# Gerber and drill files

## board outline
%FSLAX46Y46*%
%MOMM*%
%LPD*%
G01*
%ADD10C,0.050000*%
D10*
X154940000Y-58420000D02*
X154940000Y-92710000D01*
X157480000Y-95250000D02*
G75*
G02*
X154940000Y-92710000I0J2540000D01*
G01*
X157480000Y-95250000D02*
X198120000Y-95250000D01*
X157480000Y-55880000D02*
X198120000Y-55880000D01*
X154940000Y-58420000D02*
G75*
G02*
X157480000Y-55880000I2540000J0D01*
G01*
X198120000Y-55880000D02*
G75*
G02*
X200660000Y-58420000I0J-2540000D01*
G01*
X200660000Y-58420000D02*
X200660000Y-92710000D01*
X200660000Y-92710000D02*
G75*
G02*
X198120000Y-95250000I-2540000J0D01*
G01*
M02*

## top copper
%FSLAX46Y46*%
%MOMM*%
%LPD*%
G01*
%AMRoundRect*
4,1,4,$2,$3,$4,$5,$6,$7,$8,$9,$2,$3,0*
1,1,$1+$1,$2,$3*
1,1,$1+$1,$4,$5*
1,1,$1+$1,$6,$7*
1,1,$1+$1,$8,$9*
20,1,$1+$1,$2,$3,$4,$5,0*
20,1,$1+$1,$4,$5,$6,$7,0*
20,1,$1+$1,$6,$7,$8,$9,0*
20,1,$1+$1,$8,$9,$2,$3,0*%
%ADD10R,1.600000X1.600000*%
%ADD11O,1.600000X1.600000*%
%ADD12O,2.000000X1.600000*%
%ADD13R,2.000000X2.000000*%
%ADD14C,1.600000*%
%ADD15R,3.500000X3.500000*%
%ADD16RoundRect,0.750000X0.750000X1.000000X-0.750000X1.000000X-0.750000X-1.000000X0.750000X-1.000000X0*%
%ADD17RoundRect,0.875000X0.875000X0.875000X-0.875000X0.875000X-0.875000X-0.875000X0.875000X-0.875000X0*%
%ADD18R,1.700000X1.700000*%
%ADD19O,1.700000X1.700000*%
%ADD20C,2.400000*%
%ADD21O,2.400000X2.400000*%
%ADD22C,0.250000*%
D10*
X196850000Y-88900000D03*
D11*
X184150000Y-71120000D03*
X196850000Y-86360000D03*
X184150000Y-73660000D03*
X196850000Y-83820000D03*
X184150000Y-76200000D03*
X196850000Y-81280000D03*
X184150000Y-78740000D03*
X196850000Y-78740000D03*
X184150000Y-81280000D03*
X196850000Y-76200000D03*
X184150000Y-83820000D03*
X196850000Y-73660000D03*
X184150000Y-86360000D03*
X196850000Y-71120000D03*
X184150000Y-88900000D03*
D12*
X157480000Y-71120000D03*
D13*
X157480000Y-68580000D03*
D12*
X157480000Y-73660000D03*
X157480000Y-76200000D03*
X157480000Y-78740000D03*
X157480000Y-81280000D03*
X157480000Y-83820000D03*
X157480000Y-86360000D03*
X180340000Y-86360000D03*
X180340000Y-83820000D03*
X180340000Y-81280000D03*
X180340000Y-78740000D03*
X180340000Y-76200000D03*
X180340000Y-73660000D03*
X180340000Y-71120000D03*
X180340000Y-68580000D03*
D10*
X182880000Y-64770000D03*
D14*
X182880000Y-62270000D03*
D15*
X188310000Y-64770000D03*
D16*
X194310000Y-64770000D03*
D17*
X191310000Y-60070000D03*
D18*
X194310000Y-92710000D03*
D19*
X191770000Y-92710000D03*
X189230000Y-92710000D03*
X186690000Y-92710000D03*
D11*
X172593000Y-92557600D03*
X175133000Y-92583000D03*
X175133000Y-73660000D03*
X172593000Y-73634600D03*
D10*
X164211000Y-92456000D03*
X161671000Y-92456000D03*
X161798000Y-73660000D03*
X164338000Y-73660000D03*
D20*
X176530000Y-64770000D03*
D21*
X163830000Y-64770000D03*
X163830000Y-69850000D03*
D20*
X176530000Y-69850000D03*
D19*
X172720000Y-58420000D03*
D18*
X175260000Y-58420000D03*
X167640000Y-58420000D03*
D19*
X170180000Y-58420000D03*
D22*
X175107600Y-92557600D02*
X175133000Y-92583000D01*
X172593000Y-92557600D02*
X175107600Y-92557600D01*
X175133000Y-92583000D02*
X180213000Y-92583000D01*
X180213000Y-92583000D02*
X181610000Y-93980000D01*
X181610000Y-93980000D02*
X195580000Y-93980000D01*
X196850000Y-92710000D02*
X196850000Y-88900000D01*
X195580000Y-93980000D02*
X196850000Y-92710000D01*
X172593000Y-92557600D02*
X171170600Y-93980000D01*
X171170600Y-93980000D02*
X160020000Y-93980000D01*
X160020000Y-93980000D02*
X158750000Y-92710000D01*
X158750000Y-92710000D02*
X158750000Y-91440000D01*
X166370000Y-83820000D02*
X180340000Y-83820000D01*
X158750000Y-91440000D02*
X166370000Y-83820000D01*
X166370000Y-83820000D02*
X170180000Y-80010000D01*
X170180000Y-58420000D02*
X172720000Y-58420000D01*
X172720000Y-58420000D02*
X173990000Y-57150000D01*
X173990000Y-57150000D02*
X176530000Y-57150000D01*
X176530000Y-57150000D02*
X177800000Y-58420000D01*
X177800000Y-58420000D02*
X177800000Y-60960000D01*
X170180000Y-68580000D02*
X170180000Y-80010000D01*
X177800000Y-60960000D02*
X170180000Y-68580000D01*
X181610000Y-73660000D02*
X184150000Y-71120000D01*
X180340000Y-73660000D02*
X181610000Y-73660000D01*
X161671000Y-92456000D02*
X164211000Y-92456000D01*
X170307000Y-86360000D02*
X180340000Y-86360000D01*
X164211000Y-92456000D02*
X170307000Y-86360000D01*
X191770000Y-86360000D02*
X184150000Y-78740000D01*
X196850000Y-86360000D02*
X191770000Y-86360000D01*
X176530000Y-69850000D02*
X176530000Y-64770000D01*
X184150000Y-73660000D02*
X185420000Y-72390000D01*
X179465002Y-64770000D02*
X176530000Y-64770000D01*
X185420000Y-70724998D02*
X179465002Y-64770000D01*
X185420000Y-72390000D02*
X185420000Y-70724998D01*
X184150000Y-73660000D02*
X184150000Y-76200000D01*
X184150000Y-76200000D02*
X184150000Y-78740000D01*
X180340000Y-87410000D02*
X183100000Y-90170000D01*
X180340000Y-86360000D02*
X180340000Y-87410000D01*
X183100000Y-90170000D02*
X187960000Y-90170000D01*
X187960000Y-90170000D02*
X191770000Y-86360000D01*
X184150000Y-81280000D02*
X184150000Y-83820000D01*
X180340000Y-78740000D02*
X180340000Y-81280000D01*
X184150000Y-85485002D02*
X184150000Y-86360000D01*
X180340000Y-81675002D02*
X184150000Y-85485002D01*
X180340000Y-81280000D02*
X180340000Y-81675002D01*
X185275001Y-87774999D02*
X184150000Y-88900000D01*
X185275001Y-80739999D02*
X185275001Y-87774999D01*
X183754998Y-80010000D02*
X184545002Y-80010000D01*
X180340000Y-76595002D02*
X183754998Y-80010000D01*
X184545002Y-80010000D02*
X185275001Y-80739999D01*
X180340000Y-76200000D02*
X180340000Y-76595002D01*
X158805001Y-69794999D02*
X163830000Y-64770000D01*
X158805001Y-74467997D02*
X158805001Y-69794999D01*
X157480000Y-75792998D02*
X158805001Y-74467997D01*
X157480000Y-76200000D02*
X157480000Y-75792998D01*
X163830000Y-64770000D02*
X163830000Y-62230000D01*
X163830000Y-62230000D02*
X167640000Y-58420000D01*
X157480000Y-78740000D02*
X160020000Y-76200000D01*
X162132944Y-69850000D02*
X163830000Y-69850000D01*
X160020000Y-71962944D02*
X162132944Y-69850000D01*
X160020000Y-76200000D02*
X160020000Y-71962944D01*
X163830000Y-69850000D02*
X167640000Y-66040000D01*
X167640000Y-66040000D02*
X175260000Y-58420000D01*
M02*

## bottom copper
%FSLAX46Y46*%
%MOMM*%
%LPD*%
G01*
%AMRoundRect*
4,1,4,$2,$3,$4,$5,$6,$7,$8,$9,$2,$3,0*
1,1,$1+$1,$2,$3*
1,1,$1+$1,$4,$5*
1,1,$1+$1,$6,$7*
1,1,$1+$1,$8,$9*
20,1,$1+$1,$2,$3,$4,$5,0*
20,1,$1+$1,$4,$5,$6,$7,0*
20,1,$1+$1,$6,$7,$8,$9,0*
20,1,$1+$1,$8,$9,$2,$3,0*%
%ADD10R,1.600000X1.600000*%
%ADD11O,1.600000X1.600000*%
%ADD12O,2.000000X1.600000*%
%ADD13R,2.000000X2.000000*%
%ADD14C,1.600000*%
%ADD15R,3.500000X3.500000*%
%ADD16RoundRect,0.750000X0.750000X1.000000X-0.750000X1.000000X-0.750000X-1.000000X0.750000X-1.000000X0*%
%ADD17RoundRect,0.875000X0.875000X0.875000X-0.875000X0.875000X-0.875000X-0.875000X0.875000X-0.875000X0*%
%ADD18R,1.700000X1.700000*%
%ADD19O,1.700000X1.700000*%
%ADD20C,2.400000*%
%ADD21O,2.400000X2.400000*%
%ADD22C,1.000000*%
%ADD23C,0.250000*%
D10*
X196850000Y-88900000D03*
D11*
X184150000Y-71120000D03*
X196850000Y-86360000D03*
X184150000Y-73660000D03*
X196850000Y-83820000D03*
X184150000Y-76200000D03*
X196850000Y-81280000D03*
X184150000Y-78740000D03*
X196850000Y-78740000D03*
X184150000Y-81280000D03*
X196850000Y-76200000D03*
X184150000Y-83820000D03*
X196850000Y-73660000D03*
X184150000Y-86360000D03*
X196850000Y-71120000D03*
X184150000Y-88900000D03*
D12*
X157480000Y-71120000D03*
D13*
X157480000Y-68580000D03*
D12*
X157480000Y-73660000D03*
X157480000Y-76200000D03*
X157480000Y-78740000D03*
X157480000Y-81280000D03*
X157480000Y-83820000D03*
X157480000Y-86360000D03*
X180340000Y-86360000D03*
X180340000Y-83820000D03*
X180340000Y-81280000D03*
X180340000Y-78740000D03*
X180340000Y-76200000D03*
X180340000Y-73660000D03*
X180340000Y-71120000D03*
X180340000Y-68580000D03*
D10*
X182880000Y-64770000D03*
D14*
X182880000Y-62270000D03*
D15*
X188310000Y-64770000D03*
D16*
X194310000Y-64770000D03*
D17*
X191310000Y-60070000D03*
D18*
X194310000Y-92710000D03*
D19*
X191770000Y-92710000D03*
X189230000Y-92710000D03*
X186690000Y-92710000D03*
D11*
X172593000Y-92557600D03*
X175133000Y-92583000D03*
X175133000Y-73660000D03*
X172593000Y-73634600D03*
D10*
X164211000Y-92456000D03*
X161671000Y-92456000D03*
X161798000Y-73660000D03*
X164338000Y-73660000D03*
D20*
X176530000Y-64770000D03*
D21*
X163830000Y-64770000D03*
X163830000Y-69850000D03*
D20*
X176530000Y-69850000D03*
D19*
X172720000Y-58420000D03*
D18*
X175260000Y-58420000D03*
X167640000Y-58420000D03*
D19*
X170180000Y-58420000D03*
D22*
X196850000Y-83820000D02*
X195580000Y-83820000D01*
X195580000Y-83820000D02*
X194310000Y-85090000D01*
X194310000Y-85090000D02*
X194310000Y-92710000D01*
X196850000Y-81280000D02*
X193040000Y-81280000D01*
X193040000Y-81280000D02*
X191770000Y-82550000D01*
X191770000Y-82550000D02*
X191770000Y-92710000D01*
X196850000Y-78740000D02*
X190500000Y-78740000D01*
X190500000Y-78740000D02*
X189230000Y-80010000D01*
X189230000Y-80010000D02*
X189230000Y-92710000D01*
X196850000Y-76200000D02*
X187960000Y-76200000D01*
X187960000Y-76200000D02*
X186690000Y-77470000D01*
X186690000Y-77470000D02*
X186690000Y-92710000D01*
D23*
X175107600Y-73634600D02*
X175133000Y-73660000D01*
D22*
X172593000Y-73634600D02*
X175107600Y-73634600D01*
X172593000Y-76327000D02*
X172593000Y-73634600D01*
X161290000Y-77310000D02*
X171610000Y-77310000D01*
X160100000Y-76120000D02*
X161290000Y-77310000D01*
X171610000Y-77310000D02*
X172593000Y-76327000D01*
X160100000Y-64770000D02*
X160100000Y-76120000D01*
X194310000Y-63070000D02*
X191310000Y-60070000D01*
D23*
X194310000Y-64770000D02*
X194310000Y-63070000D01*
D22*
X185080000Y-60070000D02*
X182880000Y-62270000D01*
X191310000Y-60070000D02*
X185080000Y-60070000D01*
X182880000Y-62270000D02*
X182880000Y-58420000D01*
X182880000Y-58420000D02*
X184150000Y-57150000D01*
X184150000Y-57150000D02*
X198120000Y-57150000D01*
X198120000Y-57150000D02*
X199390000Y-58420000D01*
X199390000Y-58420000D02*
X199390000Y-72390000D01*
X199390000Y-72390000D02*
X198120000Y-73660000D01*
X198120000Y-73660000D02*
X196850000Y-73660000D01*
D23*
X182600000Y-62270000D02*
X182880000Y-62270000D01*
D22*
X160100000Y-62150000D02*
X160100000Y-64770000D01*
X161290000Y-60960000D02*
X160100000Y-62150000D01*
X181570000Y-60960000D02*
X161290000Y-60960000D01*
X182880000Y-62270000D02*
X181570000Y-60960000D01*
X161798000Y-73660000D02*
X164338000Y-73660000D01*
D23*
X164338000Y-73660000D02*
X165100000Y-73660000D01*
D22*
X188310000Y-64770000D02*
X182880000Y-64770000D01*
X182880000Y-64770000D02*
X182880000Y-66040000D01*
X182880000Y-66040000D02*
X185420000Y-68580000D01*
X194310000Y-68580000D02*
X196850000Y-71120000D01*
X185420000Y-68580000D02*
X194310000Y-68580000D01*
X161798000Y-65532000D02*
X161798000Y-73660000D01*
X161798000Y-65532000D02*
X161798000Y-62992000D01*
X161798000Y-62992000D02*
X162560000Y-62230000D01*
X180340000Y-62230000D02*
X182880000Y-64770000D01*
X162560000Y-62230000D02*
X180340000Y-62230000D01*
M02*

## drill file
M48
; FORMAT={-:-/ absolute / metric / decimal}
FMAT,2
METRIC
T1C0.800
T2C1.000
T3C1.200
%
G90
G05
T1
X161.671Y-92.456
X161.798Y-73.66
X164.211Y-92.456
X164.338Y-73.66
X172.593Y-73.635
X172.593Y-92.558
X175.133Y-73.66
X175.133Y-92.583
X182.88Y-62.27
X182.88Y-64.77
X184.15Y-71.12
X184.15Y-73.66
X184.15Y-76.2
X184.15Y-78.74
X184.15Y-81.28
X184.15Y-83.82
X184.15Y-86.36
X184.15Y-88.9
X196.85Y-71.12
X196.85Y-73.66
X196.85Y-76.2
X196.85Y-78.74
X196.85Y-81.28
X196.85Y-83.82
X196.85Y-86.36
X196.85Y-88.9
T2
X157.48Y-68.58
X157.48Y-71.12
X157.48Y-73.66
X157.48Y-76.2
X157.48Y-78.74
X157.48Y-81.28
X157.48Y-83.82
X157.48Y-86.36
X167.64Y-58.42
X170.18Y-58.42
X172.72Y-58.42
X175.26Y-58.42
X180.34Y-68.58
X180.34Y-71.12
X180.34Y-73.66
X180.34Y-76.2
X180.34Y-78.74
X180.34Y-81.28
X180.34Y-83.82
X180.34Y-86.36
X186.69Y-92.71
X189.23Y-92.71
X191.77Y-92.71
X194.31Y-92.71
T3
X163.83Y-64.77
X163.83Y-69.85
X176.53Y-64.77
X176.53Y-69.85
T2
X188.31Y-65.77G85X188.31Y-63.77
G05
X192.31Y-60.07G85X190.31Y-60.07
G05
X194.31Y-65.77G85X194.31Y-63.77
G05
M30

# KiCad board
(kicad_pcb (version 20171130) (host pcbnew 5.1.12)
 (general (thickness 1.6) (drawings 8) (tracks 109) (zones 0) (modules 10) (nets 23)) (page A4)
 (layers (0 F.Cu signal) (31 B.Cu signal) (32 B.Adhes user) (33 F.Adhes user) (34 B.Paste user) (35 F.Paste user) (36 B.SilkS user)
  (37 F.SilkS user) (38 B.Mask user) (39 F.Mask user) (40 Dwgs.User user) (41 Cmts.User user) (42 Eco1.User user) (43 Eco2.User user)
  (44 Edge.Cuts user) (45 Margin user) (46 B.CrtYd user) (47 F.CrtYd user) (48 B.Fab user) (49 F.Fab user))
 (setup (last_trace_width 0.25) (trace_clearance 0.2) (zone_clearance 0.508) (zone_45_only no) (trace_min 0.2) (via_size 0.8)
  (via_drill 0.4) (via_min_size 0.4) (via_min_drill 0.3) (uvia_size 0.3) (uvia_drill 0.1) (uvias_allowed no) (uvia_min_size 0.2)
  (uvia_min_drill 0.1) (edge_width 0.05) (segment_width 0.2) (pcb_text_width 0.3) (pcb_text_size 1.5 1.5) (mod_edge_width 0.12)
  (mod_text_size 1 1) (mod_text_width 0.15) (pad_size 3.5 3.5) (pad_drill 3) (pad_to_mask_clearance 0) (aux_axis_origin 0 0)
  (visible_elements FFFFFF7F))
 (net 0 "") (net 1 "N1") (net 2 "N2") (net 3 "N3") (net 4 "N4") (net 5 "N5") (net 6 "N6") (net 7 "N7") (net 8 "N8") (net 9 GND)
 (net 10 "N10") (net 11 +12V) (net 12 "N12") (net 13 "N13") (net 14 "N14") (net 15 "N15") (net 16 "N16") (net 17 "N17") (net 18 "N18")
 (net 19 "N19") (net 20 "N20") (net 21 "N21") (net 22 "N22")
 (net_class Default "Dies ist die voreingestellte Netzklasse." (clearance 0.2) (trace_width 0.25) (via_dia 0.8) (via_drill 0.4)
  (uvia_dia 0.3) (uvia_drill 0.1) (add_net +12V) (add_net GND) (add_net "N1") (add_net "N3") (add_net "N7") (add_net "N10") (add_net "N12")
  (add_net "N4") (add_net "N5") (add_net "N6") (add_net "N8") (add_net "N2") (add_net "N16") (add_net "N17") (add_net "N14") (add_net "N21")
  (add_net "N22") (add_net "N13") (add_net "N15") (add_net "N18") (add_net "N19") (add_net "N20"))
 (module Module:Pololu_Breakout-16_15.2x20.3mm (layer F.Cu) (at 196.85 88.9 180)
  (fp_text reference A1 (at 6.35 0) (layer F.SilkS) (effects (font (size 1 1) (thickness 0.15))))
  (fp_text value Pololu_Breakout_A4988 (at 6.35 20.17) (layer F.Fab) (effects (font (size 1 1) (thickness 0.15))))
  (pad 1 thru_hole rect (at 0 0 180) (size 1.6 1.6) (drill 0.8) (layers *.Cu *.Mask) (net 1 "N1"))
  (pad 9 thru_hole oval (at 12.7 17.78 180) (size 1.6 1.6) (drill 0.8) (layers *.Cu *.Mask) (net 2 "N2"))
  (pad 2 thru_hole oval (at 0 2.54 180) (size 1.6 1.6) (drill 0.8) (layers *.Cu *.Mask) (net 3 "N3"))
  (pad 10 thru_hole oval (at 12.7 15.24 180) (size 1.6 1.6) (drill 0.8) (layers *.Cu *.Mask) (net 3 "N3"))
  (pad 3 thru_hole oval (at 0 5.08 180) (size 1.6 1.6) (drill 0.8) (layers *.Cu *.Mask) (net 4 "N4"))
  (pad 11 thru_hole oval (at 12.7 12.7 180) (size 1.6 1.6) (drill 0.8) (layers *.Cu *.Mask) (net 3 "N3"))
  (pad 4 thru_hole oval (at 0 7.62 180) (size 1.6 1.6) (drill 0.8) (layers *.Cu *.Mask) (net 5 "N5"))
  (pad 12 thru_hole oval (at 12.7 10.16 180) (size 1.6 1.6) (drill 0.8) (layers *.Cu *.Mask) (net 3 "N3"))
  (pad 5 thru_hole oval (at 0 10.16 180) (size 1.6 1.6) (drill 0.8) (layers *.Cu *.Mask) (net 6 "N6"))
  (pad 13 thru_hole oval (at 12.7 7.62 180) (size 1.6 1.6) (drill 0.8) (layers *.Cu *.Mask) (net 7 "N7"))
  (pad 6 thru_hole oval (at 0 12.7 180) (size 1.6 1.6) (drill 0.8) (layers *.Cu *.Mask) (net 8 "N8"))
  (pad 14 thru_hole oval (at 12.7 5.08 180) (size 1.6 1.6) (drill 0.8) (layers *.Cu *.Mask) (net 7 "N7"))
  (pad 7 thru_hole oval (at 0 15.24 180) (size 1.6 1.6) (drill 0.8) (layers *.Cu *.Mask) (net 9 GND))
  (pad 15 thru_hole oval (at 12.7 2.54 180) (size 1.6 1.6) (drill 0.8) (layers *.Cu *.Mask) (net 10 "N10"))
  (pad 8 thru_hole oval (at 0 17.78 180) (size 1.6 1.6) (drill 0.8) (layers *.Cu *.Mask) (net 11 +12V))
  (pad 16 thru_hole oval (at 12.7 0 180) (size 1.6 1.6) (drill 0.8) (layers *.Cu *.Mask) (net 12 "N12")))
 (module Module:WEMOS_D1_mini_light (layer F.Cu) (at 157.48 68.58)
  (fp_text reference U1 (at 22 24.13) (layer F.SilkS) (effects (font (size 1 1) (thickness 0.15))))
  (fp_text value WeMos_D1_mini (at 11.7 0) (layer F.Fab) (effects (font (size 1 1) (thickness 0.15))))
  (pad 2 thru_hole oval (at 0 2.54) (size 2 1.6) (drill 1) (layers *.Cu *.Mask) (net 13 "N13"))
  (pad 1 thru_hole rect (at 0 0) (size 2 2) (drill 1) (layers *.Cu *.Mask) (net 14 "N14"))
  (pad 3 thru_hole oval (at 0 5.08) (size 2 1.6) (drill 1) (layers *.Cu *.Mask) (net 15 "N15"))
  (pad 4 thru_hole oval (at 0 7.62) (size 2 1.6) (drill 1) (layers *.Cu *.Mask) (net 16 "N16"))
  (pad 5 thru_hole oval (at 0 10.16) (size 2 1.6) (drill 1) (layers *.Cu *.Mask) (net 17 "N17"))
  (pad 6 thru_hole oval (at 0 12.7) (size 2 1.6) (drill 1) (layers *.Cu *.Mask) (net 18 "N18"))
  (pad 7 thru_hole oval (at 0 15.24) (size 2 1.6) (drill 1) (layers *.Cu *.Mask) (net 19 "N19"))
  (pad 8 thru_hole oval (at 0 17.78) (size 2 1.6) (drill 1) (layers *.Cu *.Mask) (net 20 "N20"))
  (pad 9 thru_hole oval (at 22.86 17.78) (size 2 1.6) (drill 1) (layers *.Cu *.Mask) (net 3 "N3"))
  (pad 10 thru_hole oval (at 22.86 15.24) (size 2 1.6) (drill 1) (layers *.Cu *.Mask) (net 1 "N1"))
  (pad 11 thru_hole oval (at 22.86 12.7) (size 2 1.6) (drill 1) (layers *.Cu *.Mask) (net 10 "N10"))
  (pad 12 thru_hole oval (at 22.86 10.16) (size 2 1.6) (drill 1) (layers *.Cu *.Mask) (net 10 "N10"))
  (pad 13 thru_hole oval (at 22.86 7.62) (size 2 1.6) (drill 1) (layers *.Cu *.Mask) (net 12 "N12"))
  (pad 14 thru_hole oval (at 22.86 5.08) (size 2 1.6) (drill 1) (layers *.Cu *.Mask) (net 2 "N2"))
  (pad 15 thru_hole oval (at 22.86 2.54) (size 2 1.6) (drill 1) (layers *.Cu *.Mask) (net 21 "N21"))
  (pad 16 thru_hole oval (at 22.86 0) (size 2 1.6) (drill 1) (layers *.Cu *.Mask) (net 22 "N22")))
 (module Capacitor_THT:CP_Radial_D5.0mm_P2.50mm (layer F.Cu) (at 182.88 64.77 90)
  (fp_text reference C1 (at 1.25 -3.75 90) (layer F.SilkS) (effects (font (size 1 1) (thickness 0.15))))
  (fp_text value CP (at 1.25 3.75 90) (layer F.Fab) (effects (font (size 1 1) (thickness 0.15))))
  (pad 1 thru_hole rect (at 0 0 90) (size 1.6 1.6) (drill 0.8) (layers *.Cu *.Mask) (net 11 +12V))
  (pad 2 thru_hole circle (at 2.5 0 90) (size 1.6 1.6) (drill 0.8) (layers *.Cu *.Mask) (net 9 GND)))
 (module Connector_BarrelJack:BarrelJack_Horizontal (layer F.Cu) (at 188.31 64.77 180)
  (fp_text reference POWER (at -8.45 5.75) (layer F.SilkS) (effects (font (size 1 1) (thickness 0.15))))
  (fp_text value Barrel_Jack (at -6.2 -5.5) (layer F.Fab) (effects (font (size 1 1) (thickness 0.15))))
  (pad 1 thru_hole rect (at 0 0 180) (size 3.5 3.5) (drill oval 1 3) (layers *.Cu *.Mask) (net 11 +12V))
  (pad 2 thru_hole roundrect (at -6 0 180) (size 3 3.5) (drill oval 1 3) (layers *.Cu *.Mask) (roundrect_rratio 0.25) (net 9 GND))
  (pad 3 thru_hole roundrect (at -3 4.7 180) (size 3.5 3.5) (drill oval 3 1) (layers *.Cu *.Mask) (roundrect_rratio 0.25) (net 9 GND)))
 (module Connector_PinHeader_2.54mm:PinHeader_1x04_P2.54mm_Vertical (layer F.Cu) (at 194.31 92.71 270)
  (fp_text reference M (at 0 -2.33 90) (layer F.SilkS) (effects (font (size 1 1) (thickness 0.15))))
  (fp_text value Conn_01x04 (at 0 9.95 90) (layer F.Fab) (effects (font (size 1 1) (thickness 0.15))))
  (pad 1 thru_hole rect (at 0 0 270) (size 1.7 1.7) (drill 1) (layers *.Cu *.Mask) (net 4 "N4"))
  (pad 2 thru_hole oval (at 0 2.54 270) (size 1.7 1.7) (drill 1) (layers *.Cu *.Mask) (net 5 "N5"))
  (pad 3 thru_hole oval (at 0 5.08 270) (size 1.7 1.7) (drill 1) (layers *.Cu *.Mask) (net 6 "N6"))
  (pad 4 thru_hole oval (at 0 7.62 270) (size 1.7 1.7) (drill 1) (layers *.Cu *.Mask) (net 8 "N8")))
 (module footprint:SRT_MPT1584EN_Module (layer F.Cu) (at 168.91 83.82 270)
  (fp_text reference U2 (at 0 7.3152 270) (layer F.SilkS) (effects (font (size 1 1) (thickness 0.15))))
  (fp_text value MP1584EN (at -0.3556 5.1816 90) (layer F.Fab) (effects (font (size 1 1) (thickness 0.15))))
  (pad 4 thru_hole oval (at 8.7376 -3.683) (size 1.6 1.6) (drill 0.8) (layers *.Cu B.Mask) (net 1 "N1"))
  (pad 4 thru_hole oval (at 8.763 -6.223) (size 1.6 1.6) (drill 0.8) (layers *.Cu B.Mask) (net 1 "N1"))
  (pad 2 thru_hole oval (at -10.16 -6.223) (size 1.6 1.6) (drill 0.8) (layers *.Cu B.Mask) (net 9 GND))
  (pad 2 thru_hole oval (at -10.1854 -3.683) (size 1.6 1.6) (drill 0.8) (layers *.Cu B.Mask) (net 9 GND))
  (pad 3 thru_hole rect (at 8.636 4.699) (size 1.6 1.6) (drill 0.8) (layers *.Cu B.Mask) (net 3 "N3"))
  (pad 3 thru_hole rect (at 8.636 7.239) (size 1.6 1.6) (drill 0.8) (layers *.Cu B.Mask) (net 3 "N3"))
  (pad 1 thru_hole rect (at -10.16 7.112) (size 1.6 1.6) (drill 0.8) (layers *.Cu B.Mask) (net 11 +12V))
  (pad 1 thru_hole rect (at -10.16 4.572) (size 1.6 1.6) (drill 0.8) (layers *.Cu B.Mask) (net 11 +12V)))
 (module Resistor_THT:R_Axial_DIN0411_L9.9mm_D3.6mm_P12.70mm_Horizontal (layer F.Cu) (at 176.53 64.77 180)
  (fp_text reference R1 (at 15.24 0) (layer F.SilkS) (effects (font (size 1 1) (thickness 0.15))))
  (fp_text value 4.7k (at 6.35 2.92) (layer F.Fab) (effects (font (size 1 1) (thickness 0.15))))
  (pad 1 thru_hole circle (at 0 0 180) (size 2.4 2.4) (drill 1.2) (layers *.Cu *.Mask) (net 3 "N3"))
  (pad 2 thru_hole oval (at 12.7 0 180) (size 2.4 2.4) (drill 1.2) (layers *.Cu *.Mask) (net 16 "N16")))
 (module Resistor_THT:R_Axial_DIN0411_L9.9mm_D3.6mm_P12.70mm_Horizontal (layer F.Cu) (at 176.53 69.85 180)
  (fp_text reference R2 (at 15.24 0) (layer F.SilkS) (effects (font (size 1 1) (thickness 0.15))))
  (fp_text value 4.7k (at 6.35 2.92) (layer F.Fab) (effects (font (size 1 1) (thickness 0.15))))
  (pad 2 thru_hole oval (at 12.7 0 180) (size 2.4 2.4) (drill 1.2) (layers *.Cu *.Mask) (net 17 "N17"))
  (pad 1 thru_hole circle (at 0 0 180) (size 2.4 2.4) (drill 1.2) (layers *.Cu *.Mask) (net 3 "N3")))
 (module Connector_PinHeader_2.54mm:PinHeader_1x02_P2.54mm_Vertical (layer F.Cu) (at 175.26 58.42 270)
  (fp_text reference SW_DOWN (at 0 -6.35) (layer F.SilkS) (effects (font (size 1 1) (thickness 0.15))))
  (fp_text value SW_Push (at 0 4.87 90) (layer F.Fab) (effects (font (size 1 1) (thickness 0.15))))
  (pad 2 thru_hole oval (at 0 2.54 270) (size 1.7 1.7) (drill 1) (layers *.Cu *.Mask) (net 1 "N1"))
  (pad 1 thru_hole rect (at 0 0 270) (size 1.7 1.7) (drill 1) (layers *.Cu *.Mask) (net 17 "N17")))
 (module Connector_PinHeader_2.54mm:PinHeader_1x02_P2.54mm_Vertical (layer F.Cu) (at 167.64 58.42 90)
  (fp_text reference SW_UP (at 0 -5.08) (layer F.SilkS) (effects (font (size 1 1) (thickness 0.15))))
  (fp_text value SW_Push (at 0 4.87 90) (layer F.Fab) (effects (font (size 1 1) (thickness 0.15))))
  (pad 1 thru_hole rect (at 0 0 90) (size 1.7 1.7) (drill 1) (layers *.Cu *.Mask) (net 16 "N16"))
  (pad 2 thru_hole oval (at 0 2.54 90) (size 1.7 1.7) (drill 1) (layers *.Cu *.Mask) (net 1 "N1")))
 (gr_line (start 154.94 58.42) (end 154.94 92.71) (layer Edge.Cuts) (width 0.05))
 (gr_arc (start 157.48 92.71) (end 154.94 92.71) (angle -90) (layer Edge.Cuts) (width 0.05))
 (gr_line (start 157.48 95.25) (end 198.12 95.25) (layer Edge.Cuts) (width 0.05))
 (gr_line (start 157.48 55.88) (end 198.12 55.88) (layer Edge.Cuts) (width 0.05))
 (gr_arc (start 157.48 58.42) (end 157.48 55.88) (angle -90) (layer Edge.Cuts) (width 0.05))
 (gr_arc (start 198.12 58.42) (end 200.66 58.42) (angle -90) (layer Edge.Cuts) (width 0.05))
 (gr_line (start 200.66 58.42) (end 200.66 92.71) (layer Edge.Cuts) (width 0.05))
 (gr_arc (start 198.12 92.71) (end 198.12 95.25) (angle -90) (layer Edge.Cuts) (width 0.05))
 (segment (start 175.1076 92.5576) (end 175.133 92.583) (width 0.25) (layer F.Cu) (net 1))
 (segment (start 172.593 92.5576) (end 175.1076 92.5576) (width 0.25) (layer F.Cu) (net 1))
 (segment (start 175.133 92.583) (end 180.213 92.583) (width 0.25) (layer F.Cu) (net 1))
 (segment (start 180.213 92.583) (end 181.61 93.98) (width 0.25) (layer F.Cu) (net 1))
 (segment (start 181.61 93.98) (end 195.58 93.98) (width 0.25) (layer F.Cu) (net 1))
 (segment (start 196.85 92.71) (end 196.85 88.9) (width 0.25) (layer F.Cu) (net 1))
 (segment (start 195.58 93.98) (end 196.85 92.71) (width 0.25) (layer F.Cu) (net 1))
 (segment (start 172.593 92.5576) (end 171.1706 93.98) (width 0.25) (layer F.Cu) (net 1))
 (segment (start 171.1706 93.98) (end 160.02 93.98) (width 0.25) (layer F.Cu) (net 1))
 (segment (start 160.02 93.98) (end 158.75 92.71) (width 0.25) (layer F.Cu) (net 1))
 (segment (start 158.75 92.71) (end 158.75 91.44) (width 0.25) (layer F.Cu) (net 1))
 (segment (start 166.37 83.82) (end 180.34 83.82) (width 0.25) (layer F.Cu) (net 1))
 (segment (start 158.75 91.44) (end 166.37 83.82) (width 0.25) (layer F.Cu) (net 1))
 (segment (start 166.37 83.82) (end 170.18 80.01) (width 0.25) (layer F.Cu) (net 1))
 (segment (start 170.18 58.42) (end 172.72 58.42) (width 0.25) (layer F.Cu) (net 1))
 (segment (start 172.72 58.42) (end 173.99 57.15) (width 0.25) (layer F.Cu) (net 1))
 (segment (start 173.99 57.15) (end 176.53 57.15) (width 0.25) (layer F.Cu) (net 1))
 (segment (start 176.53 57.15) (end 177.8 58.42) (width 0.25) (layer F.Cu) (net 1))
 (segment (start 177.8 58.42) (end 177.8 60.96) (width 0.25) (layer F.Cu) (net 1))
 (segment (start 170.18 68.58) (end 170.18 80.01) (width 0.25) (layer F.Cu) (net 1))
 (segment (start 177.8 60.96) (end 170.18 68.58) (width 0.25) (layer F.Cu) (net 1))
 (segment (start 181.61 73.66) (end 184.15 71.12) (width 0.25) (layer F.Cu) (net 2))
 (segment (start 180.34 73.66) (end 181.61 73.66) (width 0.25) (layer F.Cu) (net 2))
 (segment (start 161.671 92.456) (end 164.211 92.456) (width 0.25) (layer F.Cu) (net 3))
 (segment (start 170.307 86.36) (end 180.34 86.36) (width 0.25) (layer F.Cu) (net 3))
 (segment (start 164.211 92.456) (end 170.307 86.36) (width 0.25) (layer F.Cu) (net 3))
 (segment (start 191.77 86.36) (end 184.15 78.74) (width 0.25) (layer F.Cu) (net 3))
 (segment (start 196.85 86.36) (end 191.77 86.36) (width 0.25) (layer F.Cu) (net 3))
 (segment (start 176.53 69.85) (end 176.53 64.77) (width 0.25) (layer F.Cu) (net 3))
 (segment (start 184.15 73.66) (end 185.42 72.39) (width 0.25) (layer F.Cu) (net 3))
 (segment (start 179.465002 64.77) (end 176.53 64.77) (width 0.25) (layer F.Cu) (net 3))
 (segment (start 185.42 70.724998) (end 179.465002 64.77) (width 0.25) (layer F.Cu) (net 3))
 (segment (start 185.42 72.39) (end 185.42 70.724998) (width 0.25) (layer F.Cu) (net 3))
 (segment (start 184.15 73.66) (end 184.15 76.2) (width 0.25) (layer F.Cu) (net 3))
 (segment (start 184.15 76.2) (end 184.15 78.74) (width 0.25) (layer F.Cu) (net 3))
 (segment (start 180.34 87.41) (end 183.1 90.17) (width 0.25) (layer F.Cu) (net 3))
 (segment (start 180.34 86.36) (end 180.34 87.41) (width 0.25) (layer F.Cu) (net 3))
 (segment (start 183.1 90.17) (end 187.96 90.17) (width 0.25) (layer F.Cu) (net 3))
 (segment (start 187.96 90.17) (end 191.77 86.36) (width 0.25) (layer F.Cu) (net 3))
 (segment (start 196.85 83.82) (end 195.58 83.82) (width 1) (layer B.Cu) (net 4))
 (segment (start 195.58 83.82) (end 194.31 85.09) (width 1) (layer B.Cu) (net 4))
 (segment (start 194.31 85.09) (end 194.31 92.71) (width 1) (layer B.Cu) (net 4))
 (segment (start 196.85 81.28) (end 193.04 81.28) (width 1) (layer B.Cu) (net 5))
 (segment (start 193.04 81.28) (end 191.77 82.55) (width 1) (layer B.Cu) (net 5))
 (segment (start 191.77 82.55) (end 191.77 92.71) (width 1) (layer B.Cu) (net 5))
 (segment (start 196.85 78.74) (end 190.5 78.74) (width 1) (layer B.Cu) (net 6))
 (segment (start 190.5 78.74) (end 189.23 80.01) (width 1) (layer B.Cu) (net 6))
 (segment (start 189.23 80.01) (end 189.23 92.71) (width 1) (layer B.Cu) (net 6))
 (segment (start 184.15 81.28) (end 184.15 83.82) (width 0.25) (layer F.Cu) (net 7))
 (segment (start 196.85 76.2) (end 187.96 76.2) (width 1) (layer B.Cu) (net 8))
 (segment (start 187.96 76.2) (end 186.69 77.47) (width 1) (layer B.Cu) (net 8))
 (segment (start 186.69 77.47) (end 186.69 92.71) (width 1) (layer B.Cu) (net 8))
 (segment (start 180.34 78.74) (end 180.34 81.28) (width 0.25) (layer F.Cu) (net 10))
 (segment (start 184.15 85.485002) (end 184.15 86.36) (width 0.25) (layer F.Cu) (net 10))
 (segment (start 180.34 81.675002) (end 184.15 85.485002) (width 0.25) (layer F.Cu) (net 10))
 (segment (start 180.34 81.28) (end 180.34 81.675002) (width 0.25) (layer F.Cu) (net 10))
 (segment (start 185.275001 87.774999) (end 184.15 88.9) (width 0.25) (layer F.Cu) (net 12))
 (segment (start 185.275001 80.739999) (end 185.275001 87.774999) (width 0.25) (layer F.Cu) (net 12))
 (segment (start 183.754998 80.01) (end 184.545002 80.01) (width 0.25) (layer F.Cu) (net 12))
 (segment (start 180.34 76.595002) (end 183.754998 80.01) (width 0.25) (layer F.Cu) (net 12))
 (segment (start 184.545002 80.01) (end 185.275001 80.739999) (width 0.25) (layer F.Cu) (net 12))
 (segment (start 180.34 76.2) (end 180.34 76.595002) (width 0.25) (layer F.Cu) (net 12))
 (segment (start 175.1076 73.6346) (end 175.133 73.66) (width 0.25) (layer B.Cu) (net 9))
 (segment (start 172.593 73.6346) (end 175.1076 73.6346) (width 1) (layer B.Cu) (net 9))
 (segment (start 172.593 76.327) (end 172.593 73.6346) (width 1) (layer B.Cu) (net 9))
 (segment (start 161.29 77.31) (end 171.61 77.31) (width 1) (layer B.Cu) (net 9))
 (segment (start 160.1 76.12) (end 161.29 77.31) (width 1) (layer B.Cu) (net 9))
 (segment (start 171.61 77.31) (end 172.593 76.327) (width 1) (layer B.Cu) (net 9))
 (segment (start 160.1 64.77) (end 160.1 76.12) (width 1) (layer B.Cu) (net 9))
 (segment (start 194.31 63.07) (end 191.31 60.07) (width 1) (layer B.Cu) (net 9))
 (segment (start 194.31 64.77) (end 194.31 63.07) (width 0.25) (layer B.Cu) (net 9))
 (segment (start 185.08 60.07) (end 182.88 62.27) (width 1) (layer B.Cu) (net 9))
 (segment (start 191.31 60.07) (end 185.08 60.07) (width 1) (layer B.Cu) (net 9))
 (segment (start 182.88 62.27) (end 182.88 58.42) (width 1) (layer B.Cu) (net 9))
 (segment (start 182.88 58.42) (end 184.15 57.15) (width 1) (layer B.Cu) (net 9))
 (segment (start 184.15 57.15) (end 198.12 57.15) (width 1) (layer B.Cu) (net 9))
 (segment (start 198.12 57.15) (end 199.39 58.42) (width 1) (layer B.Cu) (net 9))
 (segment (start 199.39 58.42) (end 199.39 72.39) (width 1) (layer B.Cu) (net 9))
 (segment (start 199.39 72.39) (end 198.12 73.66) (width 1) (layer B.Cu) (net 9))
 (segment (start 198.12 73.66) (end 196.85 73.66) (width 1) (layer B.Cu) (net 9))
 (segment (start 182.6 62.27) (end 182.88 62.27) (width 0.25) (layer B.Cu) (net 9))
 (segment (start 160.1 62.15) (end 160.1 64.77) (width 1) (layer B.Cu) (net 9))
 (segment (start 161.29 60.96) (end 160.1 62.15) (width 1) (layer B.Cu) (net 9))
 (segment (start 181.57 60.96) (end 161.29 60.96) (width 1) (layer B.Cu) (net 9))
 (segment (start 182.88 62.27) (end 181.57 60.96) (width 1) (layer B.Cu) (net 9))
 (segment (start 161.798 73.66) (end 164.338 73.66) (width 1) (layer B.Cu) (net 11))
 (segment (start 164.338 73.66) (end 165.1 73.66) (width 0.25) (layer B.Cu) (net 11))
 (segment (start 188.31 64.77) (end 182.88 64.77) (width 1) (layer B.Cu) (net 11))
 (segment (start 182.88 64.77) (end 182.88 66.04) (width 1) (layer B.Cu) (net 11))
 (segment (start 182.88 66.04) (end 185.42 68.58) (width 1) (layer B.Cu) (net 11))
 (segment (start 194.31 68.58) (end 196.85 71.12) (width 1) (layer B.Cu) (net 11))
 (segment (start 185.42 68.58) (end 194.31 68.58) (width 1) (layer B.Cu) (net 11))
 (segment (start 161.798 65.532) (end 161.798 73.66) (width 1) (layer B.Cu) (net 11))
 (segment (start 161.798 65.532) (end 161.798 62.992) (width 1) (layer B.Cu) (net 11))
 (segment (start 161.798 62.992) (end 162.56 62.23) (width 1) (layer B.Cu) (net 11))
 (segment (start 180.34 62.23) (end 182.88 64.77) (width 1) (layer B.Cu) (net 11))
 (segment (start 162.56 62.23) (end 180.34 62.23) (width 1) (layer B.Cu) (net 11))
 (segment (start 158.805001 69.794999) (end 163.83 64.77) (width 0.25) (layer F.Cu) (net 16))
 (segment (start 158.805001 74.467997) (end 158.805001 69.794999) (width 0.25) (layer F.Cu) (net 16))
 (segment (start 157.48 75.792998) (end 158.805001 74.467997) (width 0.25) (layer F.Cu) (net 16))
 (segment (start 157.48 76.2) (end 157.48 75.792998) (width 0.25) (layer F.Cu) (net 16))
 (segment (start 163.83 64.77) (end 163.83 62.23) (width 0.25) (layer F.Cu) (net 16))
 (segment (start 163.83 62.23) (end 167.64 58.42) (width 0.25) (layer F.Cu) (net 16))
 (segment (start 157.48 78.74) (end 160.02 76.2) (width 0.25) (layer F.Cu) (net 17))
 (segment (start 162.132944 69.85) (end 163.83 69.85) (width 0.25) (layer F.Cu) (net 17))
 (segment (start 160.02 71.962944) (end 162.132944 69.85) (width 0.25) (layer F.Cu) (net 17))
 (segment (start 160.02 76.2) (end 160.02 71.962944) (width 0.25) (layer F.Cu) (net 17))
 (segment (start 163.83 69.85) (end 167.64 66.04) (width 0.25) (layer F.Cu) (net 17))
 (segment (start 167.64 66.04) (end 175.26 58.42) (width 0.25) (layer F.Cu) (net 17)))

